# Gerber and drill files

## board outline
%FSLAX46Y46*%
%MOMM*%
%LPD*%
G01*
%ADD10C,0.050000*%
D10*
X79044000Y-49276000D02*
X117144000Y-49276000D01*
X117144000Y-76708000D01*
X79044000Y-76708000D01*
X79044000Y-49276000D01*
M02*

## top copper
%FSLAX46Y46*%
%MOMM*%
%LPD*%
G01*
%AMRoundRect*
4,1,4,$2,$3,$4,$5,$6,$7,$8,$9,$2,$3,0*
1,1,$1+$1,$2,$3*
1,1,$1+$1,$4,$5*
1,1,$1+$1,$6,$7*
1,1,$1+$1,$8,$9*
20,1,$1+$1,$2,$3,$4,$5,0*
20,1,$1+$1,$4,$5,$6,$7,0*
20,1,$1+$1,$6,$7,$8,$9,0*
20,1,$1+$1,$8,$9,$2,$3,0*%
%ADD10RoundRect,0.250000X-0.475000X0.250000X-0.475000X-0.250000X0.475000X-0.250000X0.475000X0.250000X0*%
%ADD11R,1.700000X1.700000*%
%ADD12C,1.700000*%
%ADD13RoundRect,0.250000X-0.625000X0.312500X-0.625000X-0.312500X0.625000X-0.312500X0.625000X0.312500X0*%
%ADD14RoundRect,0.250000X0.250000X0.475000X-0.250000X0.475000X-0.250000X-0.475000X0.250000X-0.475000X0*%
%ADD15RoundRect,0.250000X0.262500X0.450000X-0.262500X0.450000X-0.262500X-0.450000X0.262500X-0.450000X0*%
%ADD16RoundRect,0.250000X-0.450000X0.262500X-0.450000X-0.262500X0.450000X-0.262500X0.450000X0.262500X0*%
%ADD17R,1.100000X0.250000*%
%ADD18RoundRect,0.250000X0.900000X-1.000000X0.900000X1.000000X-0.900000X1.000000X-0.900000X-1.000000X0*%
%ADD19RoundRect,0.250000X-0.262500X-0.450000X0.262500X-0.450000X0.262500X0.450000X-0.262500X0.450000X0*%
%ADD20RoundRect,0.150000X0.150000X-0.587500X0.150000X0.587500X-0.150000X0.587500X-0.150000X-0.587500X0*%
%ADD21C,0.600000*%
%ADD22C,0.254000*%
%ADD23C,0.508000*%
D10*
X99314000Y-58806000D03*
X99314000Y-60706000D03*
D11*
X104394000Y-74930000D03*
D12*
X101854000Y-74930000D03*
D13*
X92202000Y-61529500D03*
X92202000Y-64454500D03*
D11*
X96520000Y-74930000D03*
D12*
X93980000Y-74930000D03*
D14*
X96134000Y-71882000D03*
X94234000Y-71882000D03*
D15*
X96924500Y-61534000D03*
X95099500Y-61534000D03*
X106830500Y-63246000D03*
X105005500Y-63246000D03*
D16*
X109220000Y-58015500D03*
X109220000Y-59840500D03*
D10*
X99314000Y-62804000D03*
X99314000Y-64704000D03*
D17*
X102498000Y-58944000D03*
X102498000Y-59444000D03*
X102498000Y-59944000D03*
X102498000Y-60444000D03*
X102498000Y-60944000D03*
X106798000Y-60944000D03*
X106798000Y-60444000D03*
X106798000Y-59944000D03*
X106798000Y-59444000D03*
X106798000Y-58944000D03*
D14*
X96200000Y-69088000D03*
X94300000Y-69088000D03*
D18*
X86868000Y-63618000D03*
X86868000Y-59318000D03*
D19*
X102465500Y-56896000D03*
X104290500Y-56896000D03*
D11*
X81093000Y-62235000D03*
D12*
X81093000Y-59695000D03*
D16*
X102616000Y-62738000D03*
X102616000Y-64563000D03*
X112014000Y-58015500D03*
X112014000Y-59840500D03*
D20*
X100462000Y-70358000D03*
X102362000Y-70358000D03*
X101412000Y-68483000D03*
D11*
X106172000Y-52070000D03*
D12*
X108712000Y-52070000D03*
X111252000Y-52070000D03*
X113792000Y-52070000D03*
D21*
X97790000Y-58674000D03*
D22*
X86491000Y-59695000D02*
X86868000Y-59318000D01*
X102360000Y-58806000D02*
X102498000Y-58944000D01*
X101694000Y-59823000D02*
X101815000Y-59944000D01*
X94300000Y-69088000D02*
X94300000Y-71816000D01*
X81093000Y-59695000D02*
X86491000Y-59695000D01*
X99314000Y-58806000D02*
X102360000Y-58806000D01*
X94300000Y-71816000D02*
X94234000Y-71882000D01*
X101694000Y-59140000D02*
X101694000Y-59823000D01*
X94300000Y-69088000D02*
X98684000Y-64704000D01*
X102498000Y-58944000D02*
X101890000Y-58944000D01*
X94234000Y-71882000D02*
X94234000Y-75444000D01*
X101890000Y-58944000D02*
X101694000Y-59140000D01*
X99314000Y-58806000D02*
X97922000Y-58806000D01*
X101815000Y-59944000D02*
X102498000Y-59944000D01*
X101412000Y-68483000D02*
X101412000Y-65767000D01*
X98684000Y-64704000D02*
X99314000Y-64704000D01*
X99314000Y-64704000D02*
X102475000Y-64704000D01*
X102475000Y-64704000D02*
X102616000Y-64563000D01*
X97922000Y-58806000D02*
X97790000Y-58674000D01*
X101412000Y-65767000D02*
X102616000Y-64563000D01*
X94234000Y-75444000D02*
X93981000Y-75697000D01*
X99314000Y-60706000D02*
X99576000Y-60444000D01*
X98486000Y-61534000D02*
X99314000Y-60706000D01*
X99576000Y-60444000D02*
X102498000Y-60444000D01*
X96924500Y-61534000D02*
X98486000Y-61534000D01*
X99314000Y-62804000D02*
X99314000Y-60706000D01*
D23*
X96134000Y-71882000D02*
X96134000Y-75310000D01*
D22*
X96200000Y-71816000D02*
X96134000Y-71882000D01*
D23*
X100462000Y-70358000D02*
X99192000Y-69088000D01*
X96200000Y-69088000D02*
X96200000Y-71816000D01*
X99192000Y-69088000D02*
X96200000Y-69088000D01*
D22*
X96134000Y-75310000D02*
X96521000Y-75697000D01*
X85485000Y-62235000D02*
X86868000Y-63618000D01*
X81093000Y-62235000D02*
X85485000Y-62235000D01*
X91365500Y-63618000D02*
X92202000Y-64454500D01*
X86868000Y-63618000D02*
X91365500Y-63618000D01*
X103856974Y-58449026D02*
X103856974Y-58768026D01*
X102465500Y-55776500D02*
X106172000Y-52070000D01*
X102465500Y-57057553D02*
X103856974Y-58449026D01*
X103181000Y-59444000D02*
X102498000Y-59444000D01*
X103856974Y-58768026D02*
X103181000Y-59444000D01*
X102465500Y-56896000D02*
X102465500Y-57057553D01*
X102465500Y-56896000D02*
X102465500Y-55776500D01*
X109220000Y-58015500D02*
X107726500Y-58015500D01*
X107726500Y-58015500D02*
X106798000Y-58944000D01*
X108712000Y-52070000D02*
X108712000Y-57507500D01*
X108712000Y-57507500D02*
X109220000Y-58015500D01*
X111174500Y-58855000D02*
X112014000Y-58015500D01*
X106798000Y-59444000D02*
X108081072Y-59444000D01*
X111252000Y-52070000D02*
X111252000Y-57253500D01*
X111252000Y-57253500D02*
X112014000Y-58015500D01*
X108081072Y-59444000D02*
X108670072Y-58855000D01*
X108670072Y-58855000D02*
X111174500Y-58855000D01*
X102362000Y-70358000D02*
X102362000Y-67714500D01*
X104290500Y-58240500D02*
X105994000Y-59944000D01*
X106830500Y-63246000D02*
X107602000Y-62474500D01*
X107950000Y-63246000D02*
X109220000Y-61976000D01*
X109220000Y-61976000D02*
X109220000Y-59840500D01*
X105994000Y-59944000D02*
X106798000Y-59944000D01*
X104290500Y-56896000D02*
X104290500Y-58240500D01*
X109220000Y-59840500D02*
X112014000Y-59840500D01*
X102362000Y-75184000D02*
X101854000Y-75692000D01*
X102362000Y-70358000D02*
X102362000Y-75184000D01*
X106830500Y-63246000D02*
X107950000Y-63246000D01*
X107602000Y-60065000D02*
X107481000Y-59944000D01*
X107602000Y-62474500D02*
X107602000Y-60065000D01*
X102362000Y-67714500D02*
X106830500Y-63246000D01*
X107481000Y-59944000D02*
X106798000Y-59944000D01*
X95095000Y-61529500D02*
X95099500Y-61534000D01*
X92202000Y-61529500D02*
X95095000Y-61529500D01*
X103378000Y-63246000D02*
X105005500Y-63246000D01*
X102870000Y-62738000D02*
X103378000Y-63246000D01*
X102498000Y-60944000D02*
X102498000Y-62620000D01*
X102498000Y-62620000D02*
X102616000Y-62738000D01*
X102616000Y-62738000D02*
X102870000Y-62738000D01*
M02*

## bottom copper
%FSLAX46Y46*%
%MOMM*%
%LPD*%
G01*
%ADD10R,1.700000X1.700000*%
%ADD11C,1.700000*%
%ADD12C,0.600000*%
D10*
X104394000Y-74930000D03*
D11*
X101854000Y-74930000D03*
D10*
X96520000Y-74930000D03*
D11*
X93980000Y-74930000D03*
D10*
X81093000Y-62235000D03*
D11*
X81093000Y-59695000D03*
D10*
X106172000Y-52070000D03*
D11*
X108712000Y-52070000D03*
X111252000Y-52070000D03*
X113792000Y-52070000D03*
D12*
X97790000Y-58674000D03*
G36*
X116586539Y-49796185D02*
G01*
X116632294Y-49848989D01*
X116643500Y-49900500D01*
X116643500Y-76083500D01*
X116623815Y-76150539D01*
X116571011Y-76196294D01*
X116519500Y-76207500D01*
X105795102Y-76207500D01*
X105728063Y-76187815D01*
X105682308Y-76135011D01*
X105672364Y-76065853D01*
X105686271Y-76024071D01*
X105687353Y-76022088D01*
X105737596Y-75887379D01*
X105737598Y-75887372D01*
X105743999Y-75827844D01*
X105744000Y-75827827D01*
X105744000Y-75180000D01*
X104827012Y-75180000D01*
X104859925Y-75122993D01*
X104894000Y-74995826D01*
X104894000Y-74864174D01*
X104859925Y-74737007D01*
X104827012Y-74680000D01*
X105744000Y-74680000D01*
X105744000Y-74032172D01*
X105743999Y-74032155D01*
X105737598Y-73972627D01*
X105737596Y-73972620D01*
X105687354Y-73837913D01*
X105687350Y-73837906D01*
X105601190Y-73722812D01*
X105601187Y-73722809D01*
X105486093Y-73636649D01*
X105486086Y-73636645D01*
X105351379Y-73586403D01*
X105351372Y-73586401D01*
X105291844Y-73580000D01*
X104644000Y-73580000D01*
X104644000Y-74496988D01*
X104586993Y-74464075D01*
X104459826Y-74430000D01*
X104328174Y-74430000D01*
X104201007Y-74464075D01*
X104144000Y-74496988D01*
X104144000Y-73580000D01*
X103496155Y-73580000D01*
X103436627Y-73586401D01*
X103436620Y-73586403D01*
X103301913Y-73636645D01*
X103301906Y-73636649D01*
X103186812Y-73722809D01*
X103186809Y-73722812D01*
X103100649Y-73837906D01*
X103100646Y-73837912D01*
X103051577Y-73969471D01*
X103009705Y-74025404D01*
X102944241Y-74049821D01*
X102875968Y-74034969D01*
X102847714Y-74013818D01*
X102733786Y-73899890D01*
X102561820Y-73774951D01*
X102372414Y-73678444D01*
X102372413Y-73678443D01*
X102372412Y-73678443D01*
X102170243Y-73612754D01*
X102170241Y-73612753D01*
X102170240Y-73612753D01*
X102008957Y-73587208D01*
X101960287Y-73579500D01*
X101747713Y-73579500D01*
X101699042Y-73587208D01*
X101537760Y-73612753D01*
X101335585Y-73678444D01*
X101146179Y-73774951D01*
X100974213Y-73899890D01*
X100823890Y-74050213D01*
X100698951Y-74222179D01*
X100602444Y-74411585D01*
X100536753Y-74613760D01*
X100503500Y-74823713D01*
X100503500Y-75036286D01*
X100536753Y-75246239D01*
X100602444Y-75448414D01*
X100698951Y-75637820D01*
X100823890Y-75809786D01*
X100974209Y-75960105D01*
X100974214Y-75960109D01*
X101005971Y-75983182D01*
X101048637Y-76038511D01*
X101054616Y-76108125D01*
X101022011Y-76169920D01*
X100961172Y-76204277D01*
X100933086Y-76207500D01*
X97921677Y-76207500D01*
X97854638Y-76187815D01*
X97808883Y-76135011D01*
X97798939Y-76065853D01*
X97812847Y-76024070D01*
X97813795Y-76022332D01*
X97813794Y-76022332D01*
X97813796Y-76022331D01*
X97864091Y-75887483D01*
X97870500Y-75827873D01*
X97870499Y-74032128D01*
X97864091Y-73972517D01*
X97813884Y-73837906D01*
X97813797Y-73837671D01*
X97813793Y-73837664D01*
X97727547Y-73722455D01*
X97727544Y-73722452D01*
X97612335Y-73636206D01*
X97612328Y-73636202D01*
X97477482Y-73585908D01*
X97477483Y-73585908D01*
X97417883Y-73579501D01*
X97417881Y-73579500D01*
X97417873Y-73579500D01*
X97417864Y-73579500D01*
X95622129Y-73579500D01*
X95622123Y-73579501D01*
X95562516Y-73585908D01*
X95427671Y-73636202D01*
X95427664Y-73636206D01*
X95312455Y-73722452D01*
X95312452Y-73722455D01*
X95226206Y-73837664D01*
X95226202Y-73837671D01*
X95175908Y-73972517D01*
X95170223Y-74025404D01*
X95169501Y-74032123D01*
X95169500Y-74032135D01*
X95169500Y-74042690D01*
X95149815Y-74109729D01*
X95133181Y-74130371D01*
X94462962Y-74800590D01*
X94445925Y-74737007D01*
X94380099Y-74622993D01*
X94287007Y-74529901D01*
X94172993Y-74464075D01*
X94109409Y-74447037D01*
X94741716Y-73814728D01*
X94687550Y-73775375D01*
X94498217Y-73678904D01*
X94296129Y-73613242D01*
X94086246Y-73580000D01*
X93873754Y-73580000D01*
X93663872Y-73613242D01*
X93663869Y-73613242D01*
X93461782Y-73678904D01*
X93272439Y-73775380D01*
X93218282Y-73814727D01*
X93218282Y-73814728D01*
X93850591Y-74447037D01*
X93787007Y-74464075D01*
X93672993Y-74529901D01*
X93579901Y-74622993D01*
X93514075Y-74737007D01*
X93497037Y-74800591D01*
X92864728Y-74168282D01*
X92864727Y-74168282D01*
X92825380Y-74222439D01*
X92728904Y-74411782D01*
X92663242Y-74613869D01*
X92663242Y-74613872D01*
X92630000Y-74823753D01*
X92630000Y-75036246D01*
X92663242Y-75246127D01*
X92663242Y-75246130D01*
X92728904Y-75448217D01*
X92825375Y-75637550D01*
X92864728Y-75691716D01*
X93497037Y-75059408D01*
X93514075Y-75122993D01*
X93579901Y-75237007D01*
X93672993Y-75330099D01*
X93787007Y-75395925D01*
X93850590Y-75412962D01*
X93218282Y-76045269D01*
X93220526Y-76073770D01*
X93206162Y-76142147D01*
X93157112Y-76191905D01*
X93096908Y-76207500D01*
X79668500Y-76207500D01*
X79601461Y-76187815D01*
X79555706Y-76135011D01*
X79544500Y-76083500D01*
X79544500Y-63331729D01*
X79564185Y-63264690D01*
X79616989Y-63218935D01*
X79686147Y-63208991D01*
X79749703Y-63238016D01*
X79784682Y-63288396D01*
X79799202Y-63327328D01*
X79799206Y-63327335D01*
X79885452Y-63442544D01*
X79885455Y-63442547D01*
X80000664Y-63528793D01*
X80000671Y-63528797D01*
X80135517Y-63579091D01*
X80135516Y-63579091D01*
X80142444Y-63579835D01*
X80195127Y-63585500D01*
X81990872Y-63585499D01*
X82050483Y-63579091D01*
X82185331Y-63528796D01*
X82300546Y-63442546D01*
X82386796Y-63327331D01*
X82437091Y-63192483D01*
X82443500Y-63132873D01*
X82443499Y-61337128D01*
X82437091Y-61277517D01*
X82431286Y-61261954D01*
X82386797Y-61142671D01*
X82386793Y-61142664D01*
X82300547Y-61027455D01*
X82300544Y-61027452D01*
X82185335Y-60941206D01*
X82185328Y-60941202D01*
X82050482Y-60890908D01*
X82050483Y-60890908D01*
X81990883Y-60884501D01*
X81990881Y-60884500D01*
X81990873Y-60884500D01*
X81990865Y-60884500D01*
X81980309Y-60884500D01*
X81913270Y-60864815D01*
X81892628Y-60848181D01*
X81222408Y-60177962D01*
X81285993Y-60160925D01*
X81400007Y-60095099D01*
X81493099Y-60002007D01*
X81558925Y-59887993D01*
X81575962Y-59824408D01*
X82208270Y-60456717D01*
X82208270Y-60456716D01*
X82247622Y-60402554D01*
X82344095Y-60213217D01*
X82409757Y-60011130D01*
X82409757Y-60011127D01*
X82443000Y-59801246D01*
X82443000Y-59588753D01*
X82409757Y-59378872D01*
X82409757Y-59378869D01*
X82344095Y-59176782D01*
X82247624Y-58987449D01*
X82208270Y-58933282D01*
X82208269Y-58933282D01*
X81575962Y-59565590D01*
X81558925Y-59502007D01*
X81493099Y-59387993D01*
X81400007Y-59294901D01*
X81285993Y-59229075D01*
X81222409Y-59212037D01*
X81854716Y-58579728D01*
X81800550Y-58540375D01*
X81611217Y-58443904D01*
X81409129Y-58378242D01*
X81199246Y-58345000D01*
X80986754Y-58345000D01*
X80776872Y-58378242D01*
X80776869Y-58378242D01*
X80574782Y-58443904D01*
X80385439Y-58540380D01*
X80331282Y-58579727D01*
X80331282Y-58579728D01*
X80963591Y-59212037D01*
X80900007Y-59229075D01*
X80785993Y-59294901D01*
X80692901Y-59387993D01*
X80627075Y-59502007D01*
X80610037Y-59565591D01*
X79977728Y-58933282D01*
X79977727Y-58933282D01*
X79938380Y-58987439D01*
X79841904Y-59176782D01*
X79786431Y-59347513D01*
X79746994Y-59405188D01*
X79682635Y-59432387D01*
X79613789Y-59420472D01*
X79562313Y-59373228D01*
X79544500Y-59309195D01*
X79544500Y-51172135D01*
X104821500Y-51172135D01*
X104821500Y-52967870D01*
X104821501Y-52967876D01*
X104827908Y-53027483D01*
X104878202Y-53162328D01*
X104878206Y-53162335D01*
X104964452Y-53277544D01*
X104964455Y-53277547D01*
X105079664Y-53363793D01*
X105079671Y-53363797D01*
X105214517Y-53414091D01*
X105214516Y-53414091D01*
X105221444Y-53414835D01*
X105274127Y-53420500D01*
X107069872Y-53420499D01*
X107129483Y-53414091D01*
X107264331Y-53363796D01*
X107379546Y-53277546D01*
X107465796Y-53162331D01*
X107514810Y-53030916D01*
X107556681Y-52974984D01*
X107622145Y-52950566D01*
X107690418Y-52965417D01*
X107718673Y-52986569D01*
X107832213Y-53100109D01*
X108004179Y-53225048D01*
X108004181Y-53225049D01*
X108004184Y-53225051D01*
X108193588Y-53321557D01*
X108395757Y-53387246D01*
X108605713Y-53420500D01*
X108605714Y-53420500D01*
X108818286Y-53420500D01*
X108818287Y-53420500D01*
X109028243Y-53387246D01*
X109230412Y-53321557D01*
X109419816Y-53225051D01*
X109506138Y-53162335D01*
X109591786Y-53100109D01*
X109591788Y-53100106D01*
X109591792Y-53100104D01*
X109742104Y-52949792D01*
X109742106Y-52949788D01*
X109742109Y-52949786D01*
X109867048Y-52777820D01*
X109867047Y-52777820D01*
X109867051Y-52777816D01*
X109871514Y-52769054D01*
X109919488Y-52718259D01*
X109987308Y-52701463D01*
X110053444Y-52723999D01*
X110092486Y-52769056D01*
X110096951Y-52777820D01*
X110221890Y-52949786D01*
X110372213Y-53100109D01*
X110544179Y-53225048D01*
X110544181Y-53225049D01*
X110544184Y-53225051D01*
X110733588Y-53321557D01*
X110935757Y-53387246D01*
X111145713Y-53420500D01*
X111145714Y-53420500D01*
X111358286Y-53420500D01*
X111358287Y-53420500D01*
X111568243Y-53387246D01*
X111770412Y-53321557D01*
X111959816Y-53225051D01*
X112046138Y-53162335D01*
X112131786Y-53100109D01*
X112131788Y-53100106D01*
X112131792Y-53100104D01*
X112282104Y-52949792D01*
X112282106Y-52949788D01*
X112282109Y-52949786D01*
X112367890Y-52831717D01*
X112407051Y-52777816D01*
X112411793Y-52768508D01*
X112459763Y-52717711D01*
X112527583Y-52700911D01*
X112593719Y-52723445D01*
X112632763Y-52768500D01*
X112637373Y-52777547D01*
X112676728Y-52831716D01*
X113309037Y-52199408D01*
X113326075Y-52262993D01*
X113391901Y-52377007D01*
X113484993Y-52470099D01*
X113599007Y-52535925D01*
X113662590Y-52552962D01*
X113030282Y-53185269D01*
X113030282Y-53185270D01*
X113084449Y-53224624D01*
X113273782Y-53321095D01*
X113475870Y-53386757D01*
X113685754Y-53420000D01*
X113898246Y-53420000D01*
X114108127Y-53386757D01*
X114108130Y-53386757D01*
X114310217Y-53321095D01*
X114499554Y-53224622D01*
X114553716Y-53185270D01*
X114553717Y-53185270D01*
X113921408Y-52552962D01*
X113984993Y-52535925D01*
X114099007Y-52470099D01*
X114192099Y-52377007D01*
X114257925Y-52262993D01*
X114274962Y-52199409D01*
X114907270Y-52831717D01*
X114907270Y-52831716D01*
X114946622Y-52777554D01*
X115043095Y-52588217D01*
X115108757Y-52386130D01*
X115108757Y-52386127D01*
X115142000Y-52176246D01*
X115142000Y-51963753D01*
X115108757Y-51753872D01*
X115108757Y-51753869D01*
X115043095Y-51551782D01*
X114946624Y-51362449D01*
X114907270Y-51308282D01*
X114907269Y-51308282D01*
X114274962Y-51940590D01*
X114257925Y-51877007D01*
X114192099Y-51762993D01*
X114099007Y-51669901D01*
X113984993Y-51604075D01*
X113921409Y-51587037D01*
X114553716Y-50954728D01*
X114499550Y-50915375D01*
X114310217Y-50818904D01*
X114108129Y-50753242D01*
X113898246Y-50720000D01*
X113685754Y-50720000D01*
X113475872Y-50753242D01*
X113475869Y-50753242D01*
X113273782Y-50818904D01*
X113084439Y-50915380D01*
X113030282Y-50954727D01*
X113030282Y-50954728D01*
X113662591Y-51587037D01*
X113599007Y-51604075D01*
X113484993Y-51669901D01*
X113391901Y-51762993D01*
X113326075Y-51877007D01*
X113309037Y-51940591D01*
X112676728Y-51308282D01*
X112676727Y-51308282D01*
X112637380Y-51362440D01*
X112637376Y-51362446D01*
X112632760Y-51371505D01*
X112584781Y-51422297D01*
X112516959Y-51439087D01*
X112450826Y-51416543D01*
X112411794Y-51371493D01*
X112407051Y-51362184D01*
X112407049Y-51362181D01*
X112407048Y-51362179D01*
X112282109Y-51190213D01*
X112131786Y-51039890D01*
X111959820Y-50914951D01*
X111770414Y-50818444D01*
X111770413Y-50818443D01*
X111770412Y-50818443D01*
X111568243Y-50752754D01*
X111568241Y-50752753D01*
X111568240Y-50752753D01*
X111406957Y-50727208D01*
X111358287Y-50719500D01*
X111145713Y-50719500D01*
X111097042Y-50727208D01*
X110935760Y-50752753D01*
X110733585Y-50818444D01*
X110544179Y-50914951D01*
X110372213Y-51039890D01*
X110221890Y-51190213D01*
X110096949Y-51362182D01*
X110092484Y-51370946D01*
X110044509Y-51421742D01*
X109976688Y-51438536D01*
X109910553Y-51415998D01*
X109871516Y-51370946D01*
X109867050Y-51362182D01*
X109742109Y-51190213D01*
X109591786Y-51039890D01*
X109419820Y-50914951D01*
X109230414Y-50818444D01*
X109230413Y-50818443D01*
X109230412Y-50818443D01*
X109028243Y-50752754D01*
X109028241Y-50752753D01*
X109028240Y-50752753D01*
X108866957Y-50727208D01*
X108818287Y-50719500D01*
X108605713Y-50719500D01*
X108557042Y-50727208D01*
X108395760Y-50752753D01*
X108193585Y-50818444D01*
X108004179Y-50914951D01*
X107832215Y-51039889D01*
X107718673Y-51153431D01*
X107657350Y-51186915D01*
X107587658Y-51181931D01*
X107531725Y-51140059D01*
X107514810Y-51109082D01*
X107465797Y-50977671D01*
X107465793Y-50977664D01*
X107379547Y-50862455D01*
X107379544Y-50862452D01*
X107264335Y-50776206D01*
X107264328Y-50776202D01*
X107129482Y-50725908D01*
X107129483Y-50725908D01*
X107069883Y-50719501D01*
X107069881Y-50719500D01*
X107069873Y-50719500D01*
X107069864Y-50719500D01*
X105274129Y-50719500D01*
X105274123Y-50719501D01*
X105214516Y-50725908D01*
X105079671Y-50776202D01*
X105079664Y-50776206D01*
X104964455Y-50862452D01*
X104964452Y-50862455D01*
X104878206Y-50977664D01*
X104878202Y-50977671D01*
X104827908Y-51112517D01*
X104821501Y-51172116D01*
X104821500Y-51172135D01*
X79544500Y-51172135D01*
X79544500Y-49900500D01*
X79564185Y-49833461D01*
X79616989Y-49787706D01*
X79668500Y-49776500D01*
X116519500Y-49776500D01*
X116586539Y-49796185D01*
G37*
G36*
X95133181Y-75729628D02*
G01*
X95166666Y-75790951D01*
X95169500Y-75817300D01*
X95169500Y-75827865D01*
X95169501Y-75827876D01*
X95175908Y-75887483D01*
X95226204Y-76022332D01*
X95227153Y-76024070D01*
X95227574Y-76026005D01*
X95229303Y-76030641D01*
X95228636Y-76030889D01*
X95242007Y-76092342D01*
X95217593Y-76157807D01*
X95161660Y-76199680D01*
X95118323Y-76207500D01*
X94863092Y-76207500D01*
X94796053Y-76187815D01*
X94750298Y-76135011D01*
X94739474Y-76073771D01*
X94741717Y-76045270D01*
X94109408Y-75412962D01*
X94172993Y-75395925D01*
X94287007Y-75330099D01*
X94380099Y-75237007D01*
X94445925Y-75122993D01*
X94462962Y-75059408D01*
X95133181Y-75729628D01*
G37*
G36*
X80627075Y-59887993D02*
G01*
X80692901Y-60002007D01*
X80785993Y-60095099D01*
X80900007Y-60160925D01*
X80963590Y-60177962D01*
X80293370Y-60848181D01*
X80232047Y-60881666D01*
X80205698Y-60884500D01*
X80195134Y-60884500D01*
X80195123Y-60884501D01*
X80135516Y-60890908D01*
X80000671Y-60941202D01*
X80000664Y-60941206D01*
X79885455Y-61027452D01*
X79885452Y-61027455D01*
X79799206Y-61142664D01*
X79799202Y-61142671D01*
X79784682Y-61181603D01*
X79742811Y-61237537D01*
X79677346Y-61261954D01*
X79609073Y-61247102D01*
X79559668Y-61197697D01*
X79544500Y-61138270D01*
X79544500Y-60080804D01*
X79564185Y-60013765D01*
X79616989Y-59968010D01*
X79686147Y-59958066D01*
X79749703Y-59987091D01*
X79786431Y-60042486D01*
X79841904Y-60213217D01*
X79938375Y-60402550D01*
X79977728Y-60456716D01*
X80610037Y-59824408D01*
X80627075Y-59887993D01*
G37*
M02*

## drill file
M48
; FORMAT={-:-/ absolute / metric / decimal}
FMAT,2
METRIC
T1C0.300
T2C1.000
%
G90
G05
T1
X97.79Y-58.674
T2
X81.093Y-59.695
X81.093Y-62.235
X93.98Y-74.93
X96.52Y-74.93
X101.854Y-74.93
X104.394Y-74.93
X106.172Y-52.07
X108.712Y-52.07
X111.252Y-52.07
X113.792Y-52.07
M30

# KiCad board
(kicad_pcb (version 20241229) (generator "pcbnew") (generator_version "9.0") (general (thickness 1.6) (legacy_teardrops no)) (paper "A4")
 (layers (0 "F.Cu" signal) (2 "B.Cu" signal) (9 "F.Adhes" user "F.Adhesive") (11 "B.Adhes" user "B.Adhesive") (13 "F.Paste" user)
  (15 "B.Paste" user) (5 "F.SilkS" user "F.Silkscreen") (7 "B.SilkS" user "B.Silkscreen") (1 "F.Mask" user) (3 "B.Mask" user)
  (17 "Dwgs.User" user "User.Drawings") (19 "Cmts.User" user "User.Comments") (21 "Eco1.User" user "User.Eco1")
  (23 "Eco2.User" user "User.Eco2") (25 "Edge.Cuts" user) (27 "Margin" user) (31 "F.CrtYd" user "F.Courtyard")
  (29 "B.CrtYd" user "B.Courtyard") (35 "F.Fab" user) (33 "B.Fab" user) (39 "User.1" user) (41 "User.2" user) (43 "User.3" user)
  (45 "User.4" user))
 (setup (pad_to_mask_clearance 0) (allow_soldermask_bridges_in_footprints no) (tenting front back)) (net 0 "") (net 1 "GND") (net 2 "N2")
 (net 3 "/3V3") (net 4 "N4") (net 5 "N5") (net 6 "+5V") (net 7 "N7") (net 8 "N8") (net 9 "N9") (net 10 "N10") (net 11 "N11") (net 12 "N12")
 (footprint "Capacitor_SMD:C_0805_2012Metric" (layer "F.Cu") (at 99.314 59.756 -90)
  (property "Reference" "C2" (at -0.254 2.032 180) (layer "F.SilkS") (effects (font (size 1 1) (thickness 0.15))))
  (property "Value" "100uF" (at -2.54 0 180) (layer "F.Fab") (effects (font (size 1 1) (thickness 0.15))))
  (pad "1" smd roundrect (at -0.95 0 270) (size 1 1.45) (layers "F.Cu" "F.Mask" "F.Paste") (roundrect_rratio 0.25) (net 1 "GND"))
  (pad "2" smd roundrect (at 0.95 0 270) (size 1 1.45) (layers "F.Cu" "F.Mask" "F.Paste") (roundrect_rratio 0.25) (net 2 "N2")))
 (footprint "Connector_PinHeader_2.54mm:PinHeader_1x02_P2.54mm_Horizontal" (layer "F.Cu") (at 104.394 74.93 -90)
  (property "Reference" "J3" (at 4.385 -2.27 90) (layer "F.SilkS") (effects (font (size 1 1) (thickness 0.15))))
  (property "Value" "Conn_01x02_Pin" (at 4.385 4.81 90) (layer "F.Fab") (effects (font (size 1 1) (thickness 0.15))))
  (pad "1" thru_hole rect (at 0 0 270) (size 1.7 1.7) (drill 1) (layers "*.Cu" "*.Mask") (remove_unused_layers no) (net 1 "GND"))
  (pad "2" thru_hole circle (at 0 2.54 270) (size 1.7 1.7) (drill 1) (layers "*.Cu" "*.Mask") (remove_unused_layers no) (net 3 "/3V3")))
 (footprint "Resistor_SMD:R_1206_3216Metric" (layer "F.Cu") (at 92.202 62.992 -90)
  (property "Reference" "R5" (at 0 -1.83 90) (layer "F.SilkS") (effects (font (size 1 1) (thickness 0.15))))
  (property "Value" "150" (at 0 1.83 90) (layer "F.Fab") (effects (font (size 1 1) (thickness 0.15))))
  (pad "1" smd roundrect (at -1.4625 0 270) (size 1.125 1.75) (layers "F.Cu" "F.Mask" "F.Paste") (roundrect_rratio 0.222222) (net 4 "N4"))
  (pad "2" smd roundrect (at 1.4625 0 270) (size 1.125 1.75) (layers "F.Cu" "F.Mask" "F.Paste") (roundrect_rratio 0.222222) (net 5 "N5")))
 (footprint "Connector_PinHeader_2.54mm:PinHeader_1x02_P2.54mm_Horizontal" (layer "F.Cu") (at 96.52 74.93 -90)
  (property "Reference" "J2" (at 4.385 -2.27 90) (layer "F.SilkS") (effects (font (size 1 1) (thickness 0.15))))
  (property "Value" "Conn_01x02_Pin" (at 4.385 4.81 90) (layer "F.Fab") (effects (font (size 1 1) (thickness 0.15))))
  (pad "1" thru_hole rect (at 0 0 270) (size 1.7 1.7) (drill 1) (layers "*.Cu" "*.Mask") (remove_unused_layers no) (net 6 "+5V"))
  (pad "2" thru_hole circle (at 0 2.54 270) (size 1.7 1.7) (drill 1) (layers "*.Cu" "*.Mask") (remove_unused_layers no) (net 1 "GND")))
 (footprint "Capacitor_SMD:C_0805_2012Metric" (layer "F.Cu") (at 95.184 71.882 180)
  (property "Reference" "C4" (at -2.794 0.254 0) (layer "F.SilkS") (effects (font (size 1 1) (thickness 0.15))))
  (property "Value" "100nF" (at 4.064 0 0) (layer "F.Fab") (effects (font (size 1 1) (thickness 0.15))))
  (pad "1" smd roundrect (at -0.95 0 180) (size 1 1.45) (layers "F.Cu" "F.Mask" "F.Paste") (roundrect_rratio 0.25) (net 6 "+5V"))
  (pad "2" smd roundrect (at 0.95 0 180) (size 1 1.45) (layers "F.Cu" "F.Mask" "F.Paste") (roundrect_rratio 0.25) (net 1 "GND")))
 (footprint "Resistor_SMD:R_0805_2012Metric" (layer "F.Cu") (at 96.012 61.534 180)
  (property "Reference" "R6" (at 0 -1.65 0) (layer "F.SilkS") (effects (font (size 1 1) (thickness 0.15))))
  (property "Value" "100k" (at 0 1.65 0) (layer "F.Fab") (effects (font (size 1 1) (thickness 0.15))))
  (pad "1" smd roundrect (at -0.9125 0 180) (size 1.025 1.4) (layers "F.Cu" "F.Mask" "F.Paste") (roundrect_rratio 0.243902) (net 2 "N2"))
  (pad "2" smd roundrect (at 0.9125 0 180) (size 1.025 1.4) (layers "F.Cu" "F.Mask" "F.Paste") (roundrect_rratio 0.243902) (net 4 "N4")))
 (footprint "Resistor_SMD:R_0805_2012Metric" (layer "F.Cu") (at 105.918 63.246 180)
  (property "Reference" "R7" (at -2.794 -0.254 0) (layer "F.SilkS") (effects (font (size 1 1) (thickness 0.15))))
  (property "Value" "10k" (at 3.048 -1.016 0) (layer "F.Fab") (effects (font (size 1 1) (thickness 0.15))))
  (pad "1" smd roundrect (at -0.9125 0 180) (size 1.025 1.4) (layers "F.Cu" "F.Mask" "F.Paste") (roundrect_rratio 0.243902) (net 3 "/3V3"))
  (pad "2" smd roundrect (at 0.9125 0 180) (size 1.025 1.4) (layers "F.Cu" "F.Mask" "F.Paste") (roundrect_rratio 0.243902) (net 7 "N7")))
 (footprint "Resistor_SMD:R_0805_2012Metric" (layer "F.Cu") (at 109.22 58.928 -90)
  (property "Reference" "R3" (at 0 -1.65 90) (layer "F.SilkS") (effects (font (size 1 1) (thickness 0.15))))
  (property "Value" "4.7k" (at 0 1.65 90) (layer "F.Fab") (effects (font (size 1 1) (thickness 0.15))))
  (pad "1" smd roundrect (at -0.9125 0 270) (size 1.025 1.4) (layers "F.Cu" "F.Mask" "F.Paste") (roundrect_rratio 0.243902) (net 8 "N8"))
  (pad "2" smd roundrect (at 0.9125 0 270) (size 1.025 1.4) (layers "F.Cu" "F.Mask" "F.Paste") (roundrect_rratio 0.243902) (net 3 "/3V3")))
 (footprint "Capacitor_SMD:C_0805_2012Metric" (layer "F.Cu") (at 99.314 63.754 -90)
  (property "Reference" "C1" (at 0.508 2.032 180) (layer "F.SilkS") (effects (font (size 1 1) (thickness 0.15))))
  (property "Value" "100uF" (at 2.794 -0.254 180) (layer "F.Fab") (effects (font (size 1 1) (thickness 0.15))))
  (pad "1" smd roundrect (at -0.95 0 270) (size 1 1.45) (layers "F.Cu" "F.Mask" "F.Paste") (roundrect_rratio 0.25) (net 2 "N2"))
  (pad "2" smd roundrect (at 0.95 0 270) (size 1 1.45) (layers "F.Cu" "F.Mask" "F.Paste") (roundrect_rratio 0.25) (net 1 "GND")))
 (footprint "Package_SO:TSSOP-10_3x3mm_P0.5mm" (layer "F.Cu") (at 104.648 59.944)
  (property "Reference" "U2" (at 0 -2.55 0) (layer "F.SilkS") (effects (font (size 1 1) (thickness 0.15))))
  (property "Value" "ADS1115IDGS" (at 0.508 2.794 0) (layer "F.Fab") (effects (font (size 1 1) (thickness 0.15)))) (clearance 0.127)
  (pad "1" smd rect (at -2.15 -1) (size 1.1 0.25) (layers "F.Cu" "F.Mask" "F.Paste") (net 1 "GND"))
  (pad "2" smd rect (at -2.15 -0.5) (size 1.1 0.25) (layers "F.Cu" "F.Mask" "F.Paste") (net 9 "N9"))
  (pad "3" smd rect (at -2.15 0) (size 1.1 0.25) (layers "F.Cu" "F.Mask" "F.Paste") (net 1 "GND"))
  (pad "4" smd rect (at -2.15 0.5) (size 1.1 0.25) (layers "F.Cu" "F.Mask" "F.Paste") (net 2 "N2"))
  (pad "5" smd rect (at -2.15 1) (size 1.1 0.25) (layers "F.Cu" "F.Mask" "F.Paste") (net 7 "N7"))
  (pad "6" smd rect (at 2.15 1) (size 1.1 0.25) (layers "F.Cu" "F.Mask" "F.Paste") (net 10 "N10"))
  (pad "7" smd rect (at 2.15 0.5) (size 1.1 0.25) (layers "F.Cu" "F.Mask" "F.Paste") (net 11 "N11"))
  (pad "8" smd rect (at 2.15 0) (size 1.1 0.25) (layers "F.Cu" "F.Mask" "F.Paste") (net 3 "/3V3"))
  (pad "9" smd rect (at 2.15 -0.5) (size 1.1 0.25) (layers "F.Cu" "F.Mask" "F.Paste") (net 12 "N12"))
  (pad "10" smd rect (at 2.15 -1) (size 1.1 0.25) (layers "F.Cu" "F.Mask" "F.Paste") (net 8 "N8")))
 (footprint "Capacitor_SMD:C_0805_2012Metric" (layer "F.Cu") (at 95.25 69.088 180)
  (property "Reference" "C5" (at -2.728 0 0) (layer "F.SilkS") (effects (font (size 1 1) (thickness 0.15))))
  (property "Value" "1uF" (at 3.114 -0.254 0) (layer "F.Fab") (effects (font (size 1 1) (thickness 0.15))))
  (pad "1" smd roundrect (at -0.95 0 180) (size 1 1.45) (layers "F.Cu" "F.Mask" "F.Paste") (roundrect_rratio 0.25) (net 6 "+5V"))
  (pad "2" smd roundrect (at 0.95 0 180) (size 1 1.45) (layers "F.Cu" "F.Mask" "F.Paste") (roundrect_rratio 0.25) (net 1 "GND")))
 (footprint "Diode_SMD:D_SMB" (layer "F.Cu") (at 86.868 61.468 90)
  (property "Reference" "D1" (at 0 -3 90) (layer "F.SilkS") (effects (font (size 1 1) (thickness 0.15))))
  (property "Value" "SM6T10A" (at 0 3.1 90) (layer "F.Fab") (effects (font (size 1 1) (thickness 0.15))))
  (pad "1" smd roundrect (at -2.15 0 90) (size 2.5 2.3) (layers "F.Cu" "F.Mask" "F.Paste") (roundrect_rratio 0.1086956522) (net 5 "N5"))
  (pad "2" smd roundrect (at 2.15 0 90) (size 2.5 2.3) (layers "F.Cu" "F.Mask" "F.Paste") (roundrect_rratio 0.1086956522) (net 1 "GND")))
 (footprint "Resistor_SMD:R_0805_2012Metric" (layer "F.Cu") (at 103.378 56.896)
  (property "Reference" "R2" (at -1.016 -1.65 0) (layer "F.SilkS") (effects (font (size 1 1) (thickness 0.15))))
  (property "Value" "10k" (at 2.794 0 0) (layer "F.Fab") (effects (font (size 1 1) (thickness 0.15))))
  (pad "1" smd roundrect (at -0.9125 0) (size 1.025 1.4) (layers "F.Cu" "F.Mask" "F.Paste") (roundrect_rratio 0.243902) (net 9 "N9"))
  (pad "2" smd roundrect (at 0.9125 0) (size 1.025 1.4) (layers "F.Cu" "F.Mask" "F.Paste") (roundrect_rratio 0.243902) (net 3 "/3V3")))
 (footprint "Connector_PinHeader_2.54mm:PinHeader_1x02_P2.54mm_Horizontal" (layer "F.Cu") (at 81.093 62.235 180)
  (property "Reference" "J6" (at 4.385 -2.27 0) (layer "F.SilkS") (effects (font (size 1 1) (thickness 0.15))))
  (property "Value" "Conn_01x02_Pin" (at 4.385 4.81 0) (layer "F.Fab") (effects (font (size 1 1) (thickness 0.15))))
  (pad "1" thru_hole rect (at 0 0 180) (size 1.7 1.7) (drill 1) (layers "*.Cu" "*.Mask") (remove_unused_layers no) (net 5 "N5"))
  (pad "2" thru_hole circle (at 0 2.54 180) (size 1.7 1.7) (drill 1) (layers "*.Cu" "*.Mask") (remove_unused_layers no) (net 1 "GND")))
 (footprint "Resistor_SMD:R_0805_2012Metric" (layer "F.Cu") (at 102.616 63.6505 -90)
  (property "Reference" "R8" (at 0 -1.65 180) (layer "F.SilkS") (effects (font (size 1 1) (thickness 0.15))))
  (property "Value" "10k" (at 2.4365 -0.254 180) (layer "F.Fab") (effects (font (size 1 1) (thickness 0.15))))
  (pad "1" smd roundrect (at -0.9125 0 270) (size 1.025 1.4) (layers "F.Cu" "F.Mask" "F.Paste") (roundrect_rratio 0.243902) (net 7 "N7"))
  (pad "2" smd roundrect (at 0.9125 0 270) (size 1.025 1.4) (layers "F.Cu" "F.Mask" "F.Paste") (roundrect_rratio 0.243902) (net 1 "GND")))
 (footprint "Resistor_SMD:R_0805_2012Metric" (layer "F.Cu") (at 112.014 58.928 -90)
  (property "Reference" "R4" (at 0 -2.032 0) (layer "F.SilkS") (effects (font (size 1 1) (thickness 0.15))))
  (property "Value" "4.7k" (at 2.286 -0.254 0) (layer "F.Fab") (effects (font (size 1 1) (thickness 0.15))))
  (pad "1" smd roundrect (at -0.9125 0 270) (size 1.025 1.4) (layers "F.Cu" "F.Mask" "F.Paste") (roundrect_rratio 0.243902) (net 12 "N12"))
  (pad "2" smd roundrect (at 0.9125 0 270) (size 1.025 1.4) (layers "F.Cu" "F.Mask" "F.Paste") (roundrect_rratio 0.243902) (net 3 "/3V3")))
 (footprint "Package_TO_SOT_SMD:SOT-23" (layer "F.Cu") (at 101.412 69.4205 90)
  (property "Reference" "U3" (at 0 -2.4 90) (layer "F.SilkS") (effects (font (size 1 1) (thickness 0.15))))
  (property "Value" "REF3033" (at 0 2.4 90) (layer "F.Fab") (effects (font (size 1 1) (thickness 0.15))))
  (pad "1" smd roundrect (at -0.9375 -0.95 90) (size 1.475 0.6) (layers "F.Cu" "F.Mask" "F.Paste") (roundrect_rratio 0.25) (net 6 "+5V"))
  (pad "2" smd roundrect (at -0.9375 0.95 90) (size 1.475 0.6) (layers "F.Cu" "F.Mask" "F.Paste") (roundrect_rratio 0.25) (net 3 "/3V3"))
  (pad "3" smd roundrect (at 0.9375 0 90) (size 1.475 0.6) (layers "F.Cu" "F.Mask" "F.Paste") (roundrect_rratio 0.25) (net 1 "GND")))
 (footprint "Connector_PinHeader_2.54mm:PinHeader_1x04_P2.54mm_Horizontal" (layer "F.Cu") (at 106.172 52.07 90)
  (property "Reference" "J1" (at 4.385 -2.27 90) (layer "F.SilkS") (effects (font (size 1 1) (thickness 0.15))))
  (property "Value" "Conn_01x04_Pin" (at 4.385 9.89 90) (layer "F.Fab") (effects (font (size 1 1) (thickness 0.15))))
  (pad "1" thru_hole rect (at 0 0 90) (size 1.7 1.7) (drill 1) (layers "*.Cu" "*.Mask") (remove_unused_layers no) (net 9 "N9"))
  (pad "2" thru_hole circle (at 0 2.54 90) (size 1.7 1.7) (drill 1) (layers "*.Cu" "*.Mask") (remove_unused_layers no) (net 8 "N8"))
  (pad "3" thru_hole circle (at 0 5.08 90) (size 1.7 1.7) (drill 1) (layers "*.Cu" "*.Mask") (remove_unused_layers no) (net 12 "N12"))
  (pad "4" thru_hole circle (at 0 7.62 90) (size 1.7 1.7) (drill 1) (layers "*.Cu" "*.Mask") (remove_unused_layers no) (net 1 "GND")))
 (gr_rect (start 79.044 49.276) (end 117.144 76.708) (stroke (width 0.05) (type default)) (fill no) (layer "Edge.Cuts"))
 (segment (start 86.491 59.695) (end 86.868 59.318) (width 0.254) (layer "F.Cu") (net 1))
 (segment (start 102.36 58.806) (end 102.498 58.944) (width 0.254) (layer "F.Cu") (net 1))
 (segment (start 101.694 59.823) (end 101.815 59.944) (width 0.254) (layer "F.Cu") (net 1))
 (segment (start 94.3 69.088) (end 94.3 71.816) (width 0.254) (layer "F.Cu") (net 1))
 (segment (start 81.093 59.695) (end 86.491 59.695) (width 0.254) (layer "F.Cu") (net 1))
 (segment (start 99.314 58.806) (end 102.36 58.806) (width 0.254) (layer "F.Cu") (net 1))
 (segment (start 94.3 71.816) (end 94.234 71.882) (width 0.254) (layer "F.Cu") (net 1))
 (segment (start 101.694 59.14) (end 101.694 59.823) (width 0.254) (layer "F.Cu") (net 1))
 (segment (start 94.3 69.088) (end 98.684 64.704) (width 0.254) (layer "F.Cu") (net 1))
 (segment (start 102.498 58.944) (end 101.89 58.944) (width 0.254) (layer "F.Cu") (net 1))
 (segment (start 94.234 71.882) (end 94.234 75.444) (width 0.254) (layer "F.Cu") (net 1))
 (segment (start 101.89 58.944) (end 101.694 59.14) (width 0.254) (layer "F.Cu") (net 1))
 (segment (start 99.314 58.806) (end 97.922 58.806) (width 0.254) (layer "F.Cu") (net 1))
 (segment (start 101.815 59.944) (end 102.498 59.944) (width 0.254) (layer "F.Cu") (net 1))
 (segment (start 101.412 68.483) (end 101.412 65.767) (width 0.254) (layer "F.Cu") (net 1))
 (segment (start 98.684 64.704) (end 99.314 64.704) (width 0.254) (layer "F.Cu") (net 1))
 (segment (start 99.314 64.704) (end 102.475 64.704) (width 0.254) (layer "F.Cu") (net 1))
 (segment (start 102.475 64.704) (end 102.616 64.563) (width 0.254) (layer "F.Cu") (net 1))
 (segment (start 97.922 58.806) (end 97.79 58.674) (width 0.254) (layer "F.Cu") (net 1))
 (segment (start 101.412 65.767) (end 102.616 64.563) (width 0.254) (layer "F.Cu") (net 1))
 (segment (start 94.234 75.444) (end 93.981 75.697) (width 0.254) (layer "F.Cu") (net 1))
 (via (at 97.79 58.674) (size 0.6) (drill 0.3) (layers "F.Cu" "B.Cu") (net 1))
 (segment (start 99.314 60.706) (end 99.576 60.444) (width 0.254) (layer "F.Cu") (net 2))
 (segment (start 98.486 61.534) (end 99.314 60.706) (width 0.254) (layer "F.Cu") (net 2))
 (segment (start 99.576 60.444) (end 102.498 60.444) (width 0.254) (layer "F.Cu") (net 2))
 (segment (start 96.9245 61.534) (end 98.486 61.534) (width 0.254) (layer "F.Cu") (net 2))
 (segment (start 99.314 62.804) (end 99.314 60.706) (width 0.254) (layer "F.Cu") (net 2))
 (segment (start 96.134 71.882) (end 96.134 75.31) (width 0.508) (layer "F.Cu") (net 6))
 (segment (start 96.2 71.816) (end 96.134 71.882) (width 0.254) (layer "F.Cu") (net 6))
 (segment (start 100.462 70.358) (end 99.192 69.088) (width 0.508) (layer "F.Cu") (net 6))
 (segment (start 96.2 69.088) (end 96.2 71.816) (width 0.508) (layer "F.Cu") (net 6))
 (segment (start 99.192 69.088) (end 96.2 69.088) (width 0.508) (layer "F.Cu") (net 6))
 (segment (start 96.134 75.31) (end 96.521 75.697) (width 0.254) (layer "F.Cu") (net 6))
 (segment (start 85.485 62.235) (end 86.868 63.618) (width 0.254) (layer "F.Cu") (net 5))
 (segment (start 81.093 62.235) (end 85.485 62.235) (width 0.254) (layer "F.Cu") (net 5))
 (segment (start 91.3655 63.618) (end 92.202 64.4545) (width 0.254) (layer "F.Cu") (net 5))
 (segment (start 86.868 63.618) (end 91.3655 63.618) (width 0.254) (layer "F.Cu") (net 5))
 (segment (start 103.856974 58.449026) (end 103.856974 58.768026) (width 0.254) (layer "F.Cu") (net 9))
 (segment (start 102.4655 55.7765) (end 106.172 52.07) (width 0.254) (layer "F.Cu") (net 9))
 (segment (start 102.4655 57.057553) (end 103.856974 58.449026) (width 0.254) (layer "F.Cu") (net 9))
 (segment (start 103.181 59.444) (end 102.498 59.444) (width 0.254) (layer "F.Cu") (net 9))
 (segment (start 103.856974 58.768026) (end 103.181 59.444) (width 0.254) (layer "F.Cu") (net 9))
 (segment (start 102.4655 56.896) (end 102.4655 57.057553) (width 0.254) (layer "F.Cu") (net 9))
 (segment (start 102.4655 56.896) (end 102.4655 55.7765) (width 0.254) (layer "F.Cu") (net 9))
 (segment (start 109.22 58.0155) (end 107.7265 58.0155) (width 0.254) (layer "F.Cu") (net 8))
 (segment (start 107.7265 58.0155) (end 106.798 58.944) (width 0.254) (layer "F.Cu") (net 8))
 (segment (start 108.712 52.07) (end 108.712 57.5075) (width 0.254) (layer "F.Cu") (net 8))
 (segment (start 108.712 57.5075) (end 109.22 58.0155) (width 0.254) (layer "F.Cu") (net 8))
 (segment (start 111.1745 58.855) (end 112.014 58.0155) (width 0.254) (layer "F.Cu") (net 12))
 (segment (start 106.798 59.444) (end 108.081072 59.444) (width 0.254) (layer "F.Cu") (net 12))
 (segment (start 111.252 52.07) (end 111.252 57.2535) (width 0.254) (layer "F.Cu") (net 12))
 (segment (start 111.252 57.2535) (end 112.014 58.0155) (width 0.254) (layer "F.Cu") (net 12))
 (segment (start 108.081072 59.444) (end 108.670072 58.855) (width 0.254) (layer "F.Cu") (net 12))
 (segment (start 108.670072 58.855) (end 111.1745 58.855) (width 0.254) (layer "F.Cu") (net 12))
 (segment (start 102.362 70.358) (end 102.362 67.7145) (width 0.254) (layer "F.Cu") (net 3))
 (segment (start 104.2905 58.2405) (end 105.994 59.944) (width 0.254) (layer "F.Cu") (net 3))
 (segment (start 106.8305 63.246) (end 107.602 62.4745) (width 0.254) (layer "F.Cu") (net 3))
 (segment (start 107.95 63.246) (end 109.22 61.976) (width 0.254) (layer "F.Cu") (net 3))
 (segment (start 109.22 61.976) (end 109.22 59.8405) (width 0.254) (layer "F.Cu") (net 3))
 (segment (start 105.994 59.944) (end 106.798 59.944) (width 0.254) (layer "F.Cu") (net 3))
 (segment (start 104.2905 56.896) (end 104.2905 58.2405) (width 0.254) (layer "F.Cu") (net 3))
 (segment (start 109.22 59.8405) (end 112.014 59.8405) (width 0.254) (layer "F.Cu") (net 3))
 (segment (start 102.362 75.184) (end 101.854 75.692) (width 0.254) (layer "F.Cu") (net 3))
 (segment (start 102.362 70.358) (end 102.362 75.184) (width 0.254) (layer "F.Cu") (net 3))
 (segment (start 106.8305 63.246) (end 107.95 63.246) (width 0.254) (layer "F.Cu") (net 3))
 (segment (start 107.602 60.065) (end 107.481 59.944) (width 0.254) (layer "F.Cu") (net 3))
 (segment (start 107.602 62.4745) (end 107.602 60.065) (width 0.254) (layer "F.Cu") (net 3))
 (segment (start 102.362 67.7145) (end 106.8305 63.246) (width 0.254) (layer "F.Cu") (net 3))
 (segment (start 107.481 59.944) (end 106.798 59.944) (width 0.254) (layer "F.Cu") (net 3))
 (segment (start 95.095 61.5295) (end 95.0995 61.534) (width 0.254) (layer "F.Cu") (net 4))
 (segment (start 92.202 61.5295) (end 95.095 61.5295) (width 0.254) (layer "F.Cu") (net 4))
 (segment (start 103.378 63.246) (end 105.0055 63.246) (width 0.254) (layer "F.Cu") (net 7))
 (segment (start 102.87 62.738) (end 103.378 63.246) (width 0.254) (layer "F.Cu") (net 7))
 (segment (start 102.498 60.944) (end 102.498 62.62) (width 0.254) (layer "F.Cu") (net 7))
 (segment (start 102.498 62.62) (end 102.616 62.738) (width 0.254) (layer "F.Cu") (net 7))
 (segment (start 102.616 62.738) (end 102.87 62.738) (width 0.254) (layer "F.Cu") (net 7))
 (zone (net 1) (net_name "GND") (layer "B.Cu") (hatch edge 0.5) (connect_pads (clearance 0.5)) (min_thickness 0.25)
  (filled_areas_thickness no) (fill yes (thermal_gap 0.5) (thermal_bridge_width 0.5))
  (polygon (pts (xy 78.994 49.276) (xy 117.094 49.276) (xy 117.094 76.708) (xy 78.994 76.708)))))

